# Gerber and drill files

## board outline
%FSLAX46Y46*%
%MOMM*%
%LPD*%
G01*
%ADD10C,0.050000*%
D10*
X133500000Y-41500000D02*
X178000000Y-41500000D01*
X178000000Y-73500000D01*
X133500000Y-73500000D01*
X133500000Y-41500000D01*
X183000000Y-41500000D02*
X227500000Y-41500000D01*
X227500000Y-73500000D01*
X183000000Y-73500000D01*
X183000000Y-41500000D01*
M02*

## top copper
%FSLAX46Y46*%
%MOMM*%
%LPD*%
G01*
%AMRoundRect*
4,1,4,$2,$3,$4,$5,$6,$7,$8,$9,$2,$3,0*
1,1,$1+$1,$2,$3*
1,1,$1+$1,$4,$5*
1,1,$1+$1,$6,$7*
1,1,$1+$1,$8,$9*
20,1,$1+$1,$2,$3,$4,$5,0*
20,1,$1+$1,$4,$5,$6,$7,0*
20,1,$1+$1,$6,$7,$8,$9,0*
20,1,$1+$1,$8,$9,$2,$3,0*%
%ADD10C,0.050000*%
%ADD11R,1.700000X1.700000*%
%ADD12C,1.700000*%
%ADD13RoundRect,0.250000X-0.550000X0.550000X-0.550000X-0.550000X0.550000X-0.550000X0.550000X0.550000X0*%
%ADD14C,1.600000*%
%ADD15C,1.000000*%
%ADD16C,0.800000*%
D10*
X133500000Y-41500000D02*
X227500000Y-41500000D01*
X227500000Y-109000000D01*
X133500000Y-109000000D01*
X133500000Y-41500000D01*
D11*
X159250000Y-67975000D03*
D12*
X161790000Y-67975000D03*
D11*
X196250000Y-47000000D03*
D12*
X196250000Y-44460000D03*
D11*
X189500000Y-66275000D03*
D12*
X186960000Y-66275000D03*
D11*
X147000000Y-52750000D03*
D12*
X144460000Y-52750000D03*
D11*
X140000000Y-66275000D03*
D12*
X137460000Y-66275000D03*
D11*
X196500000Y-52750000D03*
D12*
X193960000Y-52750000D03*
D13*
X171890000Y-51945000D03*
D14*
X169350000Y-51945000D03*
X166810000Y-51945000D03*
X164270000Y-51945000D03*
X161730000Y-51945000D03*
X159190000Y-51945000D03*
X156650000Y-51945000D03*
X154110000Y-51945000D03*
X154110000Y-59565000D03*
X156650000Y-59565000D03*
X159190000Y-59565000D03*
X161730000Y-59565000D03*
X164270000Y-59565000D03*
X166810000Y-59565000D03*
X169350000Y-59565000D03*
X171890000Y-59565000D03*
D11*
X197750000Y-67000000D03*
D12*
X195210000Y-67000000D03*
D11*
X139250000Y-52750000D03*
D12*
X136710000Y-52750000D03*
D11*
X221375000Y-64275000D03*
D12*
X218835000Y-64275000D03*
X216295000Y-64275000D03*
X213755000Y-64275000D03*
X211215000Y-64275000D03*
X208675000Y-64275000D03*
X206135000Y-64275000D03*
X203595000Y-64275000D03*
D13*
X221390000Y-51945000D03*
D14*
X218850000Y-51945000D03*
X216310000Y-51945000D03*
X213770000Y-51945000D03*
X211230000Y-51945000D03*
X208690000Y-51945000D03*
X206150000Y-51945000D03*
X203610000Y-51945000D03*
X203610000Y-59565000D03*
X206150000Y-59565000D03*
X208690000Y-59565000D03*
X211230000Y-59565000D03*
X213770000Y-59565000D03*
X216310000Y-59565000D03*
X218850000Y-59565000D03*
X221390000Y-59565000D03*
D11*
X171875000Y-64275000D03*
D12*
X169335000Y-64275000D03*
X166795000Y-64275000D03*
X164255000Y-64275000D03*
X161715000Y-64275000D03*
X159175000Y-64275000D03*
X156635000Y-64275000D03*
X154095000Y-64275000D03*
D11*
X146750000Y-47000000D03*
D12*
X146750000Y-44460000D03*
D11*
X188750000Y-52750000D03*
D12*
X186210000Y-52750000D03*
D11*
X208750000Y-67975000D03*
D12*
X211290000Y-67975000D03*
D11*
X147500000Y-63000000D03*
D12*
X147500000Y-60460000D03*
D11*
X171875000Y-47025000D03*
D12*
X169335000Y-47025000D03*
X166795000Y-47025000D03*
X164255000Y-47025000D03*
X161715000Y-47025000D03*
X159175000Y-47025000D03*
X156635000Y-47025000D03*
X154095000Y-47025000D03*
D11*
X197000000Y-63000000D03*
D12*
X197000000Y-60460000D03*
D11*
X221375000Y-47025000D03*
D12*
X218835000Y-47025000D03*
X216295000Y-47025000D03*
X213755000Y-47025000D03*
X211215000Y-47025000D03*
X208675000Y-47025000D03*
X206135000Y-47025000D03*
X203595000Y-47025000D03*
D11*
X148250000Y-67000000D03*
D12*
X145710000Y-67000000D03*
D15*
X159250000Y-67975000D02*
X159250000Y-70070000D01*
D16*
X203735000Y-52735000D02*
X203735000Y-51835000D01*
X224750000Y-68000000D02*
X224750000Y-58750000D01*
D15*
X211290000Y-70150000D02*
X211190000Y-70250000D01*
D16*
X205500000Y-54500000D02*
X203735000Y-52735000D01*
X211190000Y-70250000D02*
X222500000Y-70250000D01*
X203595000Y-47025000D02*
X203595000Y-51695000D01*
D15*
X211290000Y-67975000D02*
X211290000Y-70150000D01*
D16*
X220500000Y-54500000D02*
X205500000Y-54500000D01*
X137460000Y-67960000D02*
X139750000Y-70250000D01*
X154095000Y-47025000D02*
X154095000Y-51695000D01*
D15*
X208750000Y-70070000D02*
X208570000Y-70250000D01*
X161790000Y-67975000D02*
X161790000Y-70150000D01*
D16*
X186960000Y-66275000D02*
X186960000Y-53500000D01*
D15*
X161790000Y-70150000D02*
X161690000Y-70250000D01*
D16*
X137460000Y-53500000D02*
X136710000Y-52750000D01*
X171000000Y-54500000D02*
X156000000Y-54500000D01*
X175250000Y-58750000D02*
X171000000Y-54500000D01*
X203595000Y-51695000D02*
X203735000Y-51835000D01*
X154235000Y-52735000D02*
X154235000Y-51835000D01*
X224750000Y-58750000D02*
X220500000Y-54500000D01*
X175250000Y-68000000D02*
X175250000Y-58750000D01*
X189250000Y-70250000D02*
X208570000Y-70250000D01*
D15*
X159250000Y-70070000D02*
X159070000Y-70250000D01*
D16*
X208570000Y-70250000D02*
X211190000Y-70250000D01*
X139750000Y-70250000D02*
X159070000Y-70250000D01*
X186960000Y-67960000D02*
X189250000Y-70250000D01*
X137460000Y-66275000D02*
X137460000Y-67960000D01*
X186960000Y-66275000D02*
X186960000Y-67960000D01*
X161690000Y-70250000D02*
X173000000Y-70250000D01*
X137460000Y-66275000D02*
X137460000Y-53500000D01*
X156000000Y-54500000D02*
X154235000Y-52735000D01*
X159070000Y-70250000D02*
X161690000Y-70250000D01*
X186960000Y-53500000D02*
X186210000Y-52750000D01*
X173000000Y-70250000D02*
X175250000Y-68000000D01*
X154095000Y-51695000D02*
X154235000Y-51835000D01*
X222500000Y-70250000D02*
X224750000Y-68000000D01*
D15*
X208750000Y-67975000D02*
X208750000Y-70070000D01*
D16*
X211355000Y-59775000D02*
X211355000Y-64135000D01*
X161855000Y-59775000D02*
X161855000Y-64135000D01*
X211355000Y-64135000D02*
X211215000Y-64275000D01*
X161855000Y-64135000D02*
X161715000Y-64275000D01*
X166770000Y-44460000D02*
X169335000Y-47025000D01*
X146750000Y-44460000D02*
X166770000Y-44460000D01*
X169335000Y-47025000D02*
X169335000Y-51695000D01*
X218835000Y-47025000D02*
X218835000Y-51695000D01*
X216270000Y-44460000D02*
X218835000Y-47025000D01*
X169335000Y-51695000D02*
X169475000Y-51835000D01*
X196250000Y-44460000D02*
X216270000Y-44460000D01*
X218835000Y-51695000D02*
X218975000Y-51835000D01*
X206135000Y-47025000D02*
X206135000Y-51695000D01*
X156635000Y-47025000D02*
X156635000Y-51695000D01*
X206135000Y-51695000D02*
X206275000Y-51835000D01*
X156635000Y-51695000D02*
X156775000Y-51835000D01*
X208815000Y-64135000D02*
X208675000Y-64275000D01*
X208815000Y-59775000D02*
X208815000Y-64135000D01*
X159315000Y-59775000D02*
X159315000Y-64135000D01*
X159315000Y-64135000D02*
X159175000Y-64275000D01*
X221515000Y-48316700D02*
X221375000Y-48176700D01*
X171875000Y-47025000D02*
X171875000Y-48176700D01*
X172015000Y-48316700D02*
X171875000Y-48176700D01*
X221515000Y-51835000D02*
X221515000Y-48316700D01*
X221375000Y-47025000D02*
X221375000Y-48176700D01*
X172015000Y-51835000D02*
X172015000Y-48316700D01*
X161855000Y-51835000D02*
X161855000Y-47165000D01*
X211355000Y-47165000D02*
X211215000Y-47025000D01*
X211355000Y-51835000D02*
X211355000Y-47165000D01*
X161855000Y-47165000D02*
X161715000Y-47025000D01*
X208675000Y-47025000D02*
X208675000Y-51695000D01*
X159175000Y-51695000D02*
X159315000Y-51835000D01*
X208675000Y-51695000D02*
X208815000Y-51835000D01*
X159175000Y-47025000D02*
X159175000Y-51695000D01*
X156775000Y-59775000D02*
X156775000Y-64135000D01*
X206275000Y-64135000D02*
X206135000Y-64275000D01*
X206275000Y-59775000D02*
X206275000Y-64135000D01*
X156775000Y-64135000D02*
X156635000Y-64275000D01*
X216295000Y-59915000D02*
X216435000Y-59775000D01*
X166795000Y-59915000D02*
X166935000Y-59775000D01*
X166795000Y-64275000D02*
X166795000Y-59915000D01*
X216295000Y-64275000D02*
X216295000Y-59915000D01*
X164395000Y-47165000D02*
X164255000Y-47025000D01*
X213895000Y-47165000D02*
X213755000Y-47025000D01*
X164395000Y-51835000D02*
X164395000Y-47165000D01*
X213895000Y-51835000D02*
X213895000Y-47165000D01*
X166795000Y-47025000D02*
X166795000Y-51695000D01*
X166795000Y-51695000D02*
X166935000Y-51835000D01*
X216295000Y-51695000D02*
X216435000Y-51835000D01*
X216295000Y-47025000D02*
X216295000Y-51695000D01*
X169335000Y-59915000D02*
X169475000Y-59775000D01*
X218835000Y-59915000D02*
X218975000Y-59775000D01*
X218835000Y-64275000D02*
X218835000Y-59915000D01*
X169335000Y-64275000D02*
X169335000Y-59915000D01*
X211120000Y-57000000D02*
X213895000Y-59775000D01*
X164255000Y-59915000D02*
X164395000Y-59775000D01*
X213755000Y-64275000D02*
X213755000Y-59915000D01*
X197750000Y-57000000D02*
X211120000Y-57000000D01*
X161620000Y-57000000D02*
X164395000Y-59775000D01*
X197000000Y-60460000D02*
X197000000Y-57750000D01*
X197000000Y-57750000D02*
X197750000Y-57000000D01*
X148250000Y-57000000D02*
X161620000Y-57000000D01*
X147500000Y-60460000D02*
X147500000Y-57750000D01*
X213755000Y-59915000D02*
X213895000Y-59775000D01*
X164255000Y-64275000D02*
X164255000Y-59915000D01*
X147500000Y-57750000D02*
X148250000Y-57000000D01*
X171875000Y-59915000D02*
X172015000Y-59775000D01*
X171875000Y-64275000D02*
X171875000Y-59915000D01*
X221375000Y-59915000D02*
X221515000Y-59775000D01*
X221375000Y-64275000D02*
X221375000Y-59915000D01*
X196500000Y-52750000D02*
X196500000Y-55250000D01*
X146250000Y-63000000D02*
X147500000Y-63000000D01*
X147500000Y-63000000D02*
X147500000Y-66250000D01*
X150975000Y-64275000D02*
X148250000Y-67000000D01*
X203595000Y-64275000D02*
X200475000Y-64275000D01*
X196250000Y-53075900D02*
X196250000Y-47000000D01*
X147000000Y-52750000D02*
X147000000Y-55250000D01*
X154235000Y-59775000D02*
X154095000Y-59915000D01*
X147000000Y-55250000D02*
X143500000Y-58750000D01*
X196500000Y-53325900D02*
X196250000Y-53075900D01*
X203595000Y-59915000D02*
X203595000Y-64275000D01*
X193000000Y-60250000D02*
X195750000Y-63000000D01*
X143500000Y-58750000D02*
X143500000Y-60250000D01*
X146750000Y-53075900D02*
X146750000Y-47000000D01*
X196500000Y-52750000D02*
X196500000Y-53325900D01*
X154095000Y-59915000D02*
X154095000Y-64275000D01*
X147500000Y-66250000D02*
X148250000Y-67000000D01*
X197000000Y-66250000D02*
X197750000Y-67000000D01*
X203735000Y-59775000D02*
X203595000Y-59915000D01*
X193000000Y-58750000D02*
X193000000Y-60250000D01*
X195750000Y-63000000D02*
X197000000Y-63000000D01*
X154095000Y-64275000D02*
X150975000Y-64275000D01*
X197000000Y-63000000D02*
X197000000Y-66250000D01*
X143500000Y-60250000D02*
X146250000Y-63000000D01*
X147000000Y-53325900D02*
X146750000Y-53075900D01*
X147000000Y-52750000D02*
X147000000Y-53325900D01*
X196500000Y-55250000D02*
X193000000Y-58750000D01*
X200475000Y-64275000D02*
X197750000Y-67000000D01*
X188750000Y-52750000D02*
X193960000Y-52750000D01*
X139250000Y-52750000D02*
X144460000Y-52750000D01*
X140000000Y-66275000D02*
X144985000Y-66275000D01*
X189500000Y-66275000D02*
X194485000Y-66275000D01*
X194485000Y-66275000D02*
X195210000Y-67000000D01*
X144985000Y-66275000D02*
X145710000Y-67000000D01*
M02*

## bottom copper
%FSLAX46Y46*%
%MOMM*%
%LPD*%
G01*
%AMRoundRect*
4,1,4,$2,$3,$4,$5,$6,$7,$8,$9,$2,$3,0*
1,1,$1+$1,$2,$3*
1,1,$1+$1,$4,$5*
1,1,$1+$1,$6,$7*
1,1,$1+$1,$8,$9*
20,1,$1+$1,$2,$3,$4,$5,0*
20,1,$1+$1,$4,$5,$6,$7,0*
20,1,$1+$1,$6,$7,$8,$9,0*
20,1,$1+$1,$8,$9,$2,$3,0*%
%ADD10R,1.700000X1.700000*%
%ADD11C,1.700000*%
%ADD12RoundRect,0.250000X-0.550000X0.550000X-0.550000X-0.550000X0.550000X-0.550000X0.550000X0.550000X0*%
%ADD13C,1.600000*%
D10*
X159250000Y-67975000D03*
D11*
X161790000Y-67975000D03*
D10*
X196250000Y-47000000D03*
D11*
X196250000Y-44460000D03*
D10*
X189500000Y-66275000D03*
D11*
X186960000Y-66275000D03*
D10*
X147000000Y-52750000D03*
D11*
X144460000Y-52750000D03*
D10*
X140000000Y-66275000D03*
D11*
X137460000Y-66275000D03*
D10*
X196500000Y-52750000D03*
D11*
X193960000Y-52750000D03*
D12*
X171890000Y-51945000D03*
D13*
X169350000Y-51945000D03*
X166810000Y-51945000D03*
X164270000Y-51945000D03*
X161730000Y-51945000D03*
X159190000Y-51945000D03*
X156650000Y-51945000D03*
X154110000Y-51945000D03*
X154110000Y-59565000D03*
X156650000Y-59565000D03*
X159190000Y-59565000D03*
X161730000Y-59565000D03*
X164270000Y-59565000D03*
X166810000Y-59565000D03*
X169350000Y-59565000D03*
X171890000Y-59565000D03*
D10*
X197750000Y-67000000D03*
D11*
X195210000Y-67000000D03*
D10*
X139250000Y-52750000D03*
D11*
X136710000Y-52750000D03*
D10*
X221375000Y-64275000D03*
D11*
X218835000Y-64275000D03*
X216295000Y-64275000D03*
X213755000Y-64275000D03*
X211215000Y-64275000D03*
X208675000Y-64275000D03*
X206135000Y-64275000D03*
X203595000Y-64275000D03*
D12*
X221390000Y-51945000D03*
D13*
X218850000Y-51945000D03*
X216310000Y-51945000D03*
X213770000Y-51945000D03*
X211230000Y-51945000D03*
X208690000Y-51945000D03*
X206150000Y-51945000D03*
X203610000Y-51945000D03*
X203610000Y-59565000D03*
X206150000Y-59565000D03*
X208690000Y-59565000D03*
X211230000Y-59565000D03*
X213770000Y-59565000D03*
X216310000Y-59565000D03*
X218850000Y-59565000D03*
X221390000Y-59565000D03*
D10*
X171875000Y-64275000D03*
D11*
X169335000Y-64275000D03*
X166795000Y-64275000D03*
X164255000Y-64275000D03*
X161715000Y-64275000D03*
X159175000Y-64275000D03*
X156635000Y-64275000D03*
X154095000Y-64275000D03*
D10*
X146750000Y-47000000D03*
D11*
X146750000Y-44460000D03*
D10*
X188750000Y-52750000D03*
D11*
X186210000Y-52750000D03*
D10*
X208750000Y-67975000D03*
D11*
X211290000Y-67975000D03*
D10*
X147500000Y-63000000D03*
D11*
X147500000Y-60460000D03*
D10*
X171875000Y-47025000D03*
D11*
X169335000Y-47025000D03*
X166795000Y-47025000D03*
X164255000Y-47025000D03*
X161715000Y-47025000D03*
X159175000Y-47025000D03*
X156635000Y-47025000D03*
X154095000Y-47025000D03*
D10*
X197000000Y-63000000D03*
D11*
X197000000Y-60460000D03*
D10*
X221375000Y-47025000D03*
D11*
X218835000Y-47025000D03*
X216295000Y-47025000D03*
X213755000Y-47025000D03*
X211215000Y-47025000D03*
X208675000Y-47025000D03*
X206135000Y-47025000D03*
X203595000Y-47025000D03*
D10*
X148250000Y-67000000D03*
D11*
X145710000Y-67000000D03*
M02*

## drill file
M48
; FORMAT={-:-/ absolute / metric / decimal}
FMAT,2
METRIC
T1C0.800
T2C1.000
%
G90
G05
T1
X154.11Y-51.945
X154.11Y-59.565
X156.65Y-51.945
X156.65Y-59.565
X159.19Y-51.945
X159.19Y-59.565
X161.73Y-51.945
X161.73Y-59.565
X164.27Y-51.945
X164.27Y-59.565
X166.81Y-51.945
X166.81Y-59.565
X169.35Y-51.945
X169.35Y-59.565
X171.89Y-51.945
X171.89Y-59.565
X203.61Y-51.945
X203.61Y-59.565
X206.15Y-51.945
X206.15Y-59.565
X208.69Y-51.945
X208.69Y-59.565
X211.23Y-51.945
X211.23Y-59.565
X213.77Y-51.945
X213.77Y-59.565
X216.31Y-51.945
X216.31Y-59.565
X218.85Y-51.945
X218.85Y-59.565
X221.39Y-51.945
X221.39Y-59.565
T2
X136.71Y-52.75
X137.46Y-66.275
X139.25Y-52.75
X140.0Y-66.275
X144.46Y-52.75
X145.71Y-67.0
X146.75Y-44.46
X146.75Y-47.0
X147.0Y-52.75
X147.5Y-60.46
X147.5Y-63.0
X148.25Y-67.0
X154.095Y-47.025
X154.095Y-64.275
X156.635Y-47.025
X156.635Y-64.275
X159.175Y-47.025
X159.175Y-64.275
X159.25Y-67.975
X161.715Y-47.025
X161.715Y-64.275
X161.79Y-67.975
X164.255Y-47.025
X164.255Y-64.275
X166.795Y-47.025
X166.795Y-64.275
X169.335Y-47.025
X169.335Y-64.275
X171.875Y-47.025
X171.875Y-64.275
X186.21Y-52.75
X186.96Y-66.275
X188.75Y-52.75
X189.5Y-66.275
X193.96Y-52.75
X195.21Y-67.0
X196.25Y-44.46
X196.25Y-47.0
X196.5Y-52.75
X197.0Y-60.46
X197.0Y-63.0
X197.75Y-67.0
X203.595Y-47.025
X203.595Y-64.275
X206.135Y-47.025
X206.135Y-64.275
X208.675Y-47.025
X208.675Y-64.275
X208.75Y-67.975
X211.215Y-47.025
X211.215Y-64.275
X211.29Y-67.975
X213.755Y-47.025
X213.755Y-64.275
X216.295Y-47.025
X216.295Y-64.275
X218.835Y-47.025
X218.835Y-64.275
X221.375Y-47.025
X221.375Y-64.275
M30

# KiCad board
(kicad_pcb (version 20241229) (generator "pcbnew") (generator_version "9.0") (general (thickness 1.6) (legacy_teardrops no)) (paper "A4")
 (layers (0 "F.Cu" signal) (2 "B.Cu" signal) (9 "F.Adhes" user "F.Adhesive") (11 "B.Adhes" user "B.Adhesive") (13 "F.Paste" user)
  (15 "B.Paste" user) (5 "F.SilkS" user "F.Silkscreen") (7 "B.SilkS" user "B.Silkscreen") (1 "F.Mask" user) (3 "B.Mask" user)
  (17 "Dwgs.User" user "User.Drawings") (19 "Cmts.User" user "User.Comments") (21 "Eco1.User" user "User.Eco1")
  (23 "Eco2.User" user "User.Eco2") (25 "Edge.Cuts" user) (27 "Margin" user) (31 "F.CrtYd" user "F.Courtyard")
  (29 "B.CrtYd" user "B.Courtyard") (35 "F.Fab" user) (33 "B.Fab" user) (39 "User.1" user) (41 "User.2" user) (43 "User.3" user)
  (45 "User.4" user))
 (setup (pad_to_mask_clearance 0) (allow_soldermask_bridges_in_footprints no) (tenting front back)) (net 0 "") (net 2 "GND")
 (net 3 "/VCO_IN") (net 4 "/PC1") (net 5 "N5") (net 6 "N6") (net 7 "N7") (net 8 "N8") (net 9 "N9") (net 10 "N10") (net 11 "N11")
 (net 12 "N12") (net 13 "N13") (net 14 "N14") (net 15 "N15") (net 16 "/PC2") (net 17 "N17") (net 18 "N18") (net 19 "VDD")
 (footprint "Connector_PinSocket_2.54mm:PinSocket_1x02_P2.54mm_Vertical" (layer "F.Cu") (at 159.25 67.975 90)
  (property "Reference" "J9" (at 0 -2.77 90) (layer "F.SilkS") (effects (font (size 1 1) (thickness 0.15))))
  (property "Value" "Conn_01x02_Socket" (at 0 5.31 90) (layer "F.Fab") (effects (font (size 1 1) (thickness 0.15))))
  (pad "1" thru_hole rect (at 0 0 90) (size 1.7 1.7) (drill 1) (layers "*.Cu" "*.Mask") (remove_unused_layers no) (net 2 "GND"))
  (pad "2" thru_hole circle (at 0 2.54 90) (size 1.7 1.7) (drill 1) (layers "*.Cu" "*.Mask") (remove_unused_layers no) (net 2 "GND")))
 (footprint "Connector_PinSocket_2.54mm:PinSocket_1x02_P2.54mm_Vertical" (layer "F.Cu") (at 196.25 47 180)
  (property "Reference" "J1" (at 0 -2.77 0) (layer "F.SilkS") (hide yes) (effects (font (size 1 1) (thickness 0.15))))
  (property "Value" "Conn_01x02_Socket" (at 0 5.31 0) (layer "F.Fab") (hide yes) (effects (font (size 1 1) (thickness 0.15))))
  (pad "1" thru_hole rect (at 0 0 180) (size 1.7 1.7) (drill 1) (layers "*.Cu" "*.Mask") (remove_unused_layers no) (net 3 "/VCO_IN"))
  (pad "2" thru_hole circle (at 0 2.54 180) (size 1.7 1.7) (drill 1) (layers "*.Cu" "*.Mask") (remove_unused_layers no) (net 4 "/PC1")))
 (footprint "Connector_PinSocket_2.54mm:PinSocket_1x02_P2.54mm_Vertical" (layer "F.Cu") (at 189.5 66.275 -90)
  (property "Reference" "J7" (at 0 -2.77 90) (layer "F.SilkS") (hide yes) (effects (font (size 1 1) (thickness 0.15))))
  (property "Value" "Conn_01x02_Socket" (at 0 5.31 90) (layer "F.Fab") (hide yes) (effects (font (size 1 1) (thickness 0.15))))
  (pad "1" thru_hole rect (at 0 0 270) (size 1.7 1.7) (drill 1) (layers "*.Cu" "*.Mask") (remove_unused_layers no) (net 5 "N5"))
  (pad "2" thru_hole circle (at 0 2.54 270) (size 1.7 1.7) (drill 1) (layers "*.Cu" "*.Mask") (remove_unused_layers no) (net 2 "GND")))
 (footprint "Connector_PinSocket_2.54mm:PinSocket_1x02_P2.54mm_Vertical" (layer "F.Cu") (at 147 52.75 -90)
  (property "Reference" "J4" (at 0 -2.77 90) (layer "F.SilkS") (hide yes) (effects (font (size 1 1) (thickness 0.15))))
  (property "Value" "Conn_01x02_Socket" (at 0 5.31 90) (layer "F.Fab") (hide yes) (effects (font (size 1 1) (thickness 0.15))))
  (pad "1" thru_hole rect (at 0 0 270) (size 1.7 1.7) (drill 1) (layers "*.Cu" "*.Mask") (remove_unused_layers no) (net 3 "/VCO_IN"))
  (pad "2" thru_hole circle (at 0 2.54 270) (size 1.7 1.7) (drill 1) (layers "*.Cu" "*.Mask") (remove_unused_layers no) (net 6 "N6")))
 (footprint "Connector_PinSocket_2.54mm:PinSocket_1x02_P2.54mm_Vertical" (layer "F.Cu") (at 140 66.275 -90)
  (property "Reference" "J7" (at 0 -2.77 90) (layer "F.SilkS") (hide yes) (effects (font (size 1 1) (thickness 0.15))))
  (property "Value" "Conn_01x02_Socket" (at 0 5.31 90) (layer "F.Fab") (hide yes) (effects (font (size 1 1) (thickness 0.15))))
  (pad "1" thru_hole rect (at 0 0 270) (size 1.7 1.7) (drill 1) (layers "*.Cu" "*.Mask") (remove_unused_layers no) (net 5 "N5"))
  (pad "2" thru_hole circle (at 0 2.54 270) (size 1.7 1.7) (drill 1) (layers "*.Cu" "*.Mask") (remove_unused_layers no) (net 2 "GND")))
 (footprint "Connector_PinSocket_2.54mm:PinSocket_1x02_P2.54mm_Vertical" (layer "F.Cu") (at 196.5 52.75 -90)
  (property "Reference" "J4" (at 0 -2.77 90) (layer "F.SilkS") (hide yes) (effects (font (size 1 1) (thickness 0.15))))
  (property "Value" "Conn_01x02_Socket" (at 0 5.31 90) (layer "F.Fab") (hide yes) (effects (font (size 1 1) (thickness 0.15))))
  (pad "1" thru_hole rect (at 0 0 270) (size 1.7 1.7) (drill 1) (layers "*.Cu" "*.Mask") (remove_unused_layers no) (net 3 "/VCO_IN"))
  (pad "2" thru_hole circle (at 0 2.54 270) (size 1.7 1.7) (drill 1) (layers "*.Cu" "*.Mask") (remove_unused_layers no) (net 6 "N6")))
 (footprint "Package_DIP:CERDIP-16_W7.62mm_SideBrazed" (layer "F.Cu") (at 171.89 51.945 -90)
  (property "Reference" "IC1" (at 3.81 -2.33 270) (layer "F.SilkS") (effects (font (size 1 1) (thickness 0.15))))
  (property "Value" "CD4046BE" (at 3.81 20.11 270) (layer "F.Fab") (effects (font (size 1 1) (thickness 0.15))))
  (pad "1" thru_hole roundrect (at 0 0 270) (size 1.6 1.6) (drill 0.8) (layers "*.Cu" "*.Mask") (remove_unused_layers no)
   (roundrect_rratio 0.15625) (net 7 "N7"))
  (pad "2" thru_hole circle (at 0 2.54 270) (size 1.6 1.6) (drill 0.8) (layers "*.Cu" "*.Mask") (remove_unused_layers no) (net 4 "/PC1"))
  (pad "3" thru_hole circle (at 0 5.08 270) (size 1.6 1.6) (drill 0.8) (layers "*.Cu" "*.Mask") (remove_unused_layers no) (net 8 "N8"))
  (pad "4" thru_hole circle (at 0 7.62 270) (size 1.6 1.6) (drill 0.8) (layers "*.Cu" "*.Mask") (remove_unused_layers no) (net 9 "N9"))
  (pad "5" thru_hole circle (at 0 10.16 270) (size 1.6 1.6) (drill 0.8) (layers "*.Cu" "*.Mask") (remove_unused_layers no) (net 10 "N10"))
  (pad "6" thru_hole circle (at 0 12.7 270) (size 1.6 1.6) (drill 0.8) (layers "*.Cu" "*.Mask") (remove_unused_layers no) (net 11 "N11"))
  (pad "7" thru_hole circle (at 0 15.24 270) (size 1.6 1.6) (drill 0.8) (layers "*.Cu" "*.Mask") (remove_unused_layers no) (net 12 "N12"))
  (pad "8" thru_hole circle (at 0 17.78 270) (size 1.6 1.6) (drill 0.8) (layers "*.Cu" "*.Mask") (remove_unused_layers no) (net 2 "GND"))
  (pad "9" thru_hole circle (at 7.62 17.78 270) (size 1.6 1.6) (drill 0.8) (layers "*.Cu" "*.Mask") (remove_unused_layers no)
   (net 3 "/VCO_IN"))
  (pad "10" thru_hole circle (at 7.62 15.24 270) (size 1.6 1.6) (drill 0.8) (layers "*.Cu" "*.Mask") (remove_unused_layers no)
   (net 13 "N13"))
  (pad "11" thru_hole circle (at 7.62 12.7 270) (size 1.6 1.6) (drill 0.8) (layers "*.Cu" "*.Mask") (remove_unused_layers no) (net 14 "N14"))
  (pad "12" thru_hole circle (at 7.62 10.16 270) (size 1.6 1.6) (drill 0.8) (layers "*.Cu" "*.Mask") (remove_unused_layers no)
   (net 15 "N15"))
  (pad "13" thru_hole circle (at 7.62 7.62 270) (size 1.6 1.6) (drill 0.8) (layers "*.Cu" "*.Mask") (remove_unused_layers no)
   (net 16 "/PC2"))
  (pad "14" thru_hole circle (at 7.62 5.08 270) (size 1.6 1.6) (drill 0.8) (layers "*.Cu" "*.Mask") (remove_unused_layers no) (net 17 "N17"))
  (pad "15" thru_hole circle (at 7.62 2.54 270) (size 1.6 1.6) (drill 0.8) (layers "*.Cu" "*.Mask") (remove_unused_layers no) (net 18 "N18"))
  (pad "16" thru_hole circle (at 7.62 0 270) (size 1.6 1.6) (drill 0.8) (layers "*.Cu" "*.Mask") (remove_unused_layers no) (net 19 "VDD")))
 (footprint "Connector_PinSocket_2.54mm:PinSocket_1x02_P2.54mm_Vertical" (layer "F.Cu") (at 197.75 67 -90)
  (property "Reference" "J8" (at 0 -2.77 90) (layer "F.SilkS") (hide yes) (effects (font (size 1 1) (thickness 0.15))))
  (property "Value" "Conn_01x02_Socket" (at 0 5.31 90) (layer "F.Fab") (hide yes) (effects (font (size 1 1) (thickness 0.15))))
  (pad "1" thru_hole rect (at 0 0 270) (size 1.7 1.7) (drill 1) (layers "*.Cu" "*.Mask") (remove_unused_layers no) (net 3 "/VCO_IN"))
  (pad "2" thru_hole circle (at 0 2.54 270) (size 1.7 1.7) (drill 1) (layers "*.Cu" "*.Mask") (remove_unused_layers no) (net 5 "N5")))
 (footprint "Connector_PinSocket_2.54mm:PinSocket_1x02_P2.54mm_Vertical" (layer "F.Cu") (at 139.25 52.75 -90)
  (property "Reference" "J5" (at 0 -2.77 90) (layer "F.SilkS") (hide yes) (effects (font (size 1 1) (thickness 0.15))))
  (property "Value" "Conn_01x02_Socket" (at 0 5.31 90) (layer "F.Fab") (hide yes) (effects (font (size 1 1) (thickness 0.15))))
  (pad "1" thru_hole rect (at 0 0 270) (size 1.7 1.7) (drill 1) (layers "*.Cu" "*.Mask") (remove_unused_layers no) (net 6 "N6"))
  (pad "2" thru_hole circle (at 0 2.54 270) (size 1.7 1.7) (drill 1) (layers "*.Cu" "*.Mask") (remove_unused_layers no) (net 2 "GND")))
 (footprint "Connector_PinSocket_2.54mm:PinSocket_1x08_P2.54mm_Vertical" (layer "F.Cu") (at 221.375 64.275 -90)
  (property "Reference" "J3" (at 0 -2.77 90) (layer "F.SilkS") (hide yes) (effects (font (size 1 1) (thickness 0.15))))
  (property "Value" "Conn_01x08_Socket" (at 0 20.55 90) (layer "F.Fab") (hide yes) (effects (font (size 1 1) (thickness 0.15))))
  (pad "1" thru_hole rect (at 0 0 270) (size 1.7 1.7) (drill 1) (layers "*.Cu" "*.Mask") (remove_unused_layers no) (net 19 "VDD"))
  (pad "2" thru_hole circle (at 0 2.54 270) (size 1.7 1.7) (drill 1) (layers "*.Cu" "*.Mask") (remove_unused_layers no) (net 18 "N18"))
  (pad "3" thru_hole circle (at 0 5.08 270) (size 1.7 1.7) (drill 1) (layers "*.Cu" "*.Mask") (remove_unused_layers no) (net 17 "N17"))
  (pad "4" thru_hole circle (at 0 7.62 270) (size 1.7 1.7) (drill 1) (layers "*.Cu" "*.Mask") (remove_unused_layers no) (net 16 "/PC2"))
  (pad "5" thru_hole circle (at 0 10.16 270) (size 1.7 1.7) (drill 1) (layers "*.Cu" "*.Mask") (remove_unused_layers no) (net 15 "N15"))
  (pad "6" thru_hole circle (at 0 12.7 270) (size 1.7 1.7) (drill 1) (layers "*.Cu" "*.Mask") (remove_unused_layers no) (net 14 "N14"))
  (pad "7" thru_hole circle (at 0 15.24 270) (size 1.7 1.7) (drill 1) (layers "*.Cu" "*.Mask") (remove_unused_layers no) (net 13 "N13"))
  (pad "8" thru_hole circle (at 0 17.78 270) (size 1.7 1.7) (drill 1) (layers "*.Cu" "*.Mask") (remove_unused_layers no) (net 3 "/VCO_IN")))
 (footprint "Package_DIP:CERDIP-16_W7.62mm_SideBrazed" (layer "F.Cu") (at 221.39 51.945 -90)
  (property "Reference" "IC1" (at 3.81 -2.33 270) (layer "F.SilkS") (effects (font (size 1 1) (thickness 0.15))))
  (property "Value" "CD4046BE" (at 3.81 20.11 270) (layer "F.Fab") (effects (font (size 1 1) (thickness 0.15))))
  (pad "1" thru_hole roundrect (at 0 0 270) (size 1.6 1.6) (drill 0.8) (layers "*.Cu" "*.Mask") (remove_unused_layers no)
   (roundrect_rratio 0.15625) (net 7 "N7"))
  (pad "2" thru_hole circle (at 0 2.54 270) (size 1.6 1.6) (drill 0.8) (layers "*.Cu" "*.Mask") (remove_unused_layers no) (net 4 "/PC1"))
  (pad "3" thru_hole circle (at 0 5.08 270) (size 1.6 1.6) (drill 0.8) (layers "*.Cu" "*.Mask") (remove_unused_layers no) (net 8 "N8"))
  (pad "4" thru_hole circle (at 0 7.62 270) (size 1.6 1.6) (drill 0.8) (layers "*.Cu" "*.Mask") (remove_unused_layers no) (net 9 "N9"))
  (pad "5" thru_hole circle (at 0 10.16 270) (size 1.6 1.6) (drill 0.8) (layers "*.Cu" "*.Mask") (remove_unused_layers no) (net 10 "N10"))
  (pad "6" thru_hole circle (at 0 12.7 270) (size 1.6 1.6) (drill 0.8) (layers "*.Cu" "*.Mask") (remove_unused_layers no) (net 11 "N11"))
  (pad "7" thru_hole circle (at 0 15.24 270) (size 1.6 1.6) (drill 0.8) (layers "*.Cu" "*.Mask") (remove_unused_layers no) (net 12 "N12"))
  (pad "8" thru_hole circle (at 0 17.78 270) (size 1.6 1.6) (drill 0.8) (layers "*.Cu" "*.Mask") (remove_unused_layers no) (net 2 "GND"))
  (pad "9" thru_hole circle (at 7.62 17.78 270) (size 1.6 1.6) (drill 0.8) (layers "*.Cu" "*.Mask") (remove_unused_layers no)
   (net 3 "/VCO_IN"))
  (pad "10" thru_hole circle (at 7.62 15.24 270) (size 1.6 1.6) (drill 0.8) (layers "*.Cu" "*.Mask") (remove_unused_layers no)
   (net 13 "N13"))
  (pad "11" thru_hole circle (at 7.62 12.7 270) (size 1.6 1.6) (drill 0.8) (layers "*.Cu" "*.Mask") (remove_unused_layers no) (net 14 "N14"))
  (pad "12" thru_hole circle (at 7.62 10.16 270) (size 1.6 1.6) (drill 0.8) (layers "*.Cu" "*.Mask") (remove_unused_layers no)
   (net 15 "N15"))
  (pad "13" thru_hole circle (at 7.62 7.62 270) (size 1.6 1.6) (drill 0.8) (layers "*.Cu" "*.Mask") (remove_unused_layers no)
   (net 16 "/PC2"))
  (pad "14" thru_hole circle (at 7.62 5.08 270) (size 1.6 1.6) (drill 0.8) (layers "*.Cu" "*.Mask") (remove_unused_layers no) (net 17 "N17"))
  (pad "15" thru_hole circle (at 7.62 2.54 270) (size 1.6 1.6) (drill 0.8) (layers "*.Cu" "*.Mask") (remove_unused_layers no) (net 18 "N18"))
  (pad "16" thru_hole circle (at 7.62 0 270) (size 1.6 1.6) (drill 0.8) (layers "*.Cu" "*.Mask") (remove_unused_layers no) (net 19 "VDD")))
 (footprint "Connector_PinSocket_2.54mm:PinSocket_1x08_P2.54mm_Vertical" (layer "F.Cu") (at 171.875 64.275 -90)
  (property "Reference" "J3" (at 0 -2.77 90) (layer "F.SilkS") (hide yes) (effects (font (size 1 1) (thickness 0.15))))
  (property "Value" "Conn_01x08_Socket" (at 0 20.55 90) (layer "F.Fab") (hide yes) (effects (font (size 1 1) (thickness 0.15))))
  (pad "1" thru_hole rect (at 0 0 270) (size 1.7 1.7) (drill 1) (layers "*.Cu" "*.Mask") (remove_unused_layers no) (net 19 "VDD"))
  (pad "2" thru_hole circle (at 0 2.54 270) (size 1.7 1.7) (drill 1) (layers "*.Cu" "*.Mask") (remove_unused_layers no) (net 18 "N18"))
  (pad "3" thru_hole circle (at 0 5.08 270) (size 1.7 1.7) (drill 1) (layers "*.Cu" "*.Mask") (remove_unused_layers no) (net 17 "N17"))
  (pad "4" thru_hole circle (at 0 7.62 270) (size 1.7 1.7) (drill 1) (layers "*.Cu" "*.Mask") (remove_unused_layers no) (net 16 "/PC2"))
  (pad "5" thru_hole circle (at 0 10.16 270) (size 1.7 1.7) (drill 1) (layers "*.Cu" "*.Mask") (remove_unused_layers no) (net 15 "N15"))
  (pad "6" thru_hole circle (at 0 12.7 270) (size 1.7 1.7) (drill 1) (layers "*.Cu" "*.Mask") (remove_unused_layers no) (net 14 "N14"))
  (pad "7" thru_hole circle (at 0 15.24 270) (size 1.7 1.7) (drill 1) (layers "*.Cu" "*.Mask") (remove_unused_layers no) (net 13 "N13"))
  (pad "8" thru_hole circle (at 0 17.78 270) (size 1.7 1.7) (drill 1) (layers "*.Cu" "*.Mask") (remove_unused_layers no) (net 3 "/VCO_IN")))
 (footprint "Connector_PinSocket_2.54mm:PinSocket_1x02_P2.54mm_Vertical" (layer "F.Cu") (at 146.75 47 180)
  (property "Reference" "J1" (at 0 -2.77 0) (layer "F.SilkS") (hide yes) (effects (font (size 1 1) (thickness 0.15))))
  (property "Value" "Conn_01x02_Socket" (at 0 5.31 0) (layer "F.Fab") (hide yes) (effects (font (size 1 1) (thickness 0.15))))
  (pad "1" thru_hole rect (at 0 0 180) (size 1.7 1.7) (drill 1) (layers "*.Cu" "*.Mask") (remove_unused_layers no) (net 3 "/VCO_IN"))
  (pad "2" thru_hole circle (at 0 2.54 180) (size 1.7 1.7) (drill 1) (layers "*.Cu" "*.Mask") (remove_unused_layers no) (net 4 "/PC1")))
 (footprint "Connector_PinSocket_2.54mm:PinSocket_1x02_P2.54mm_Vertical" (layer "F.Cu") (at 188.75 52.75 -90)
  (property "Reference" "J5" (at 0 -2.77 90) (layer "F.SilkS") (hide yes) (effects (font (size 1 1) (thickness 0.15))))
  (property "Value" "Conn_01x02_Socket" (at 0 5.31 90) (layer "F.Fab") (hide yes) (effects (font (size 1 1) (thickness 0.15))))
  (pad "1" thru_hole rect (at 0 0 270) (size 1.7 1.7) (drill 1) (layers "*.Cu" "*.Mask") (remove_unused_layers no) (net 6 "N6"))
  (pad "2" thru_hole circle (at 0 2.54 270) (size 1.7 1.7) (drill 1) (layers "*.Cu" "*.Mask") (remove_unused_layers no) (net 2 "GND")))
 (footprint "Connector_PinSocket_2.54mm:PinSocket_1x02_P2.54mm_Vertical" (layer "F.Cu") (at 208.75 67.975 90)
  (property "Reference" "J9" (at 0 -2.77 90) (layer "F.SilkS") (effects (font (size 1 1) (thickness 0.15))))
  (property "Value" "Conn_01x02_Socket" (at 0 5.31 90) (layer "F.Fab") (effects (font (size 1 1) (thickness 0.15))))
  (pad "1" thru_hole rect (at 0 0 90) (size 1.7 1.7) (drill 1) (layers "*.Cu" "*.Mask") (remove_unused_layers no) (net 2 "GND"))
  (pad "2" thru_hole circle (at 0 2.54 90) (size 1.7 1.7) (drill 1) (layers "*.Cu" "*.Mask") (remove_unused_layers no) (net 2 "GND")))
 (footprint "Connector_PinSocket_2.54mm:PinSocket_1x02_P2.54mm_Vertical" (layer "F.Cu") (at 147.5 63 180)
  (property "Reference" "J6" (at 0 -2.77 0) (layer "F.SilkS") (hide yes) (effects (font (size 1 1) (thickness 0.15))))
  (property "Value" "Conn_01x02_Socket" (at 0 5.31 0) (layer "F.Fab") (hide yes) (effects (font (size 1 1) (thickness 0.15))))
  (pad "1" thru_hole rect (at 0 0 180) (size 1.7 1.7) (drill 1) (layers "*.Cu" "*.Mask") (remove_unused_layers no) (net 3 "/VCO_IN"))
  (pad "2" thru_hole circle (at 0 2.54 180) (size 1.7 1.7) (drill 1) (layers "*.Cu" "*.Mask") (remove_unused_layers no) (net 16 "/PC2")))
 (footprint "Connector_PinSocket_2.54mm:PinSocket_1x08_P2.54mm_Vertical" (layer "F.Cu") (at 171.875 47.025 -90)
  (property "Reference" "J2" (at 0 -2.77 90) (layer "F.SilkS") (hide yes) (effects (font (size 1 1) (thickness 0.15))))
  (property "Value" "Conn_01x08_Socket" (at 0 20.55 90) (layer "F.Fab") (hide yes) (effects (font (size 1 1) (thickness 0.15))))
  (pad "1" thru_hole rect (at 0 0 270) (size 1.7 1.7) (drill 1) (layers "*.Cu" "*.Mask") (remove_unused_layers no) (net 7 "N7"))
  (pad "2" thru_hole circle (at 0 2.54 270) (size 1.7 1.7) (drill 1) (layers "*.Cu" "*.Mask") (remove_unused_layers no) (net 4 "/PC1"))
  (pad "3" thru_hole circle (at 0 5.08 270) (size 1.7 1.7) (drill 1) (layers "*.Cu" "*.Mask") (remove_unused_layers no) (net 8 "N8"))
  (pad "4" thru_hole circle (at 0 7.62 270) (size 1.7 1.7) (drill 1) (layers "*.Cu" "*.Mask") (remove_unused_layers no) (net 9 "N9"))
  (pad "5" thru_hole circle (at 0 10.16 270) (size 1.7 1.7) (drill 1) (layers "*.Cu" "*.Mask") (remove_unused_layers no) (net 10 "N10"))
  (pad "6" thru_hole circle (at 0 12.7 270) (size 1.7 1.7) (drill 1) (layers "*.Cu" "*.Mask") (remove_unused_layers no) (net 11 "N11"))
  (pad "7" thru_hole circle (at 0 15.24 270) (size 1.7 1.7) (drill 1) (layers "*.Cu" "*.Mask") (remove_unused_layers no) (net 12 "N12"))
  (pad "8" thru_hole circle (at 0 17.78 270) (size 1.7 1.7) (drill 1) (layers "*.Cu" "*.Mask") (remove_unused_layers no) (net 2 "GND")))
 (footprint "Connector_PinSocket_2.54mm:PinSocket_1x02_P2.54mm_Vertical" (layer "F.Cu") (at 197 63 180)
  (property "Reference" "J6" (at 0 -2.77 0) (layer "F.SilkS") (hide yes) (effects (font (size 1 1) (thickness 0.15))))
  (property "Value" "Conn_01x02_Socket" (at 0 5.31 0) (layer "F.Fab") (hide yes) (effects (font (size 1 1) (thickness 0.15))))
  (pad "1" thru_hole rect (at 0 0 180) (size 1.7 1.7) (drill 1) (layers "*.Cu" "*.Mask") (remove_unused_layers no) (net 3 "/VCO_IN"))
  (pad "2" thru_hole circle (at 0 2.54 180) (size 1.7 1.7) (drill 1) (layers "*.Cu" "*.Mask") (remove_unused_layers no) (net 16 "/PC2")))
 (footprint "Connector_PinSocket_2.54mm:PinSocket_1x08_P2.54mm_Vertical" (layer "F.Cu") (at 221.375 47.025 -90)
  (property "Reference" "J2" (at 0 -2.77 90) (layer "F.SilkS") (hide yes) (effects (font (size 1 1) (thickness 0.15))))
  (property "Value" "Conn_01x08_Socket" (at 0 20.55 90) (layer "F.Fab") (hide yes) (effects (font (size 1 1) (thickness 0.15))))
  (pad "1" thru_hole rect (at 0 0 270) (size 1.7 1.7) (drill 1) (layers "*.Cu" "*.Mask") (remove_unused_layers no) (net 7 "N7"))
  (pad "2" thru_hole circle (at 0 2.54 270) (size 1.7 1.7) (drill 1) (layers "*.Cu" "*.Mask") (remove_unused_layers no) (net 4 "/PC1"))
  (pad "3" thru_hole circle (at 0 5.08 270) (size 1.7 1.7) (drill 1) (layers "*.Cu" "*.Mask") (remove_unused_layers no) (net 8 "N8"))
  (pad "4" thru_hole circle (at 0 7.62 270) (size 1.7 1.7) (drill 1) (layers "*.Cu" "*.Mask") (remove_unused_layers no) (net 9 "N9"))
  (pad "5" thru_hole circle (at 0 10.16 270) (size 1.7 1.7) (drill 1) (layers "*.Cu" "*.Mask") (remove_unused_layers no) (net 10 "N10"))
  (pad "6" thru_hole circle (at 0 12.7 270) (size 1.7 1.7) (drill 1) (layers "*.Cu" "*.Mask") (remove_unused_layers no) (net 11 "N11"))
  (pad "7" thru_hole circle (at 0 15.24 270) (size 1.7 1.7) (drill 1) (layers "*.Cu" "*.Mask") (remove_unused_layers no) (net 12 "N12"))
  (pad "8" thru_hole circle (at 0 17.78 270) (size 1.7 1.7) (drill 1) (layers "*.Cu" "*.Mask") (remove_unused_layers no) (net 2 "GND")))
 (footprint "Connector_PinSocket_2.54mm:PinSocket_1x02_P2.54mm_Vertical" (layer "F.Cu") (at 148.25 67 -90)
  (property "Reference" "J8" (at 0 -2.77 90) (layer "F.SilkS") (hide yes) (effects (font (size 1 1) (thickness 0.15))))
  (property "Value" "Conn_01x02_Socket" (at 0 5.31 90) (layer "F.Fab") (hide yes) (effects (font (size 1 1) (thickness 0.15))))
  (pad "1" thru_hole rect (at 0 0 270) (size 1.7 1.7) (drill 1) (layers "*.Cu" "*.Mask") (remove_unused_layers no) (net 3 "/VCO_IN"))
  (pad "2" thru_hole circle (at 0 2.54 270) (size 1.7 1.7) (drill 1) (layers "*.Cu" "*.Mask") (remove_unused_layers no) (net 5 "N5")))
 (gr_rect (start 133.5 41.5) (end 227.5 109) (stroke (width 0.05) (type solid)) (fill no) (layer "F.Cu"))
 (gr_rect (start 133.5 41.5) (end 178 73.5) (stroke (width 0.05) (type default)) (fill no) (layer "Edge.Cuts"))
 (gr_rect (start 183 41.5) (end 227.5 73.5) (stroke (width 0.05) (type default)) (fill no) (layer "Edge.Cuts"))
 (segment (start 159.25 67.975) (end 159.25 70.07) (width 1) (layer "F.Cu") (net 2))
 (segment (start 203.735 52.735) (end 203.735 51.835) (width 0.8) (layer "F.Cu") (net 2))
 (segment (start 224.75 68) (end 224.75 58.75) (width 0.8) (layer "F.Cu") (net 2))
 (segment (start 211.29 70.15) (end 211.19 70.25) (width 1) (layer "F.Cu") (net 2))
 (segment (start 205.5 54.5) (end 203.735 52.735) (width 0.8) (layer "F.Cu") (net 2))
 (segment (start 211.19 70.25) (end 222.5 70.25) (width 0.8) (layer "F.Cu") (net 2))
 (segment (start 203.595 47.025) (end 203.595 51.695) (width 0.8) (layer "F.Cu") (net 2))
 (segment (start 211.29 67.975) (end 211.29 70.15) (width 1) (layer "F.Cu") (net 2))
 (segment (start 220.5 54.5) (end 205.5 54.5) (width 0.8) (layer "F.Cu") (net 2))
 (segment (start 137.46 67.96) (end 139.75 70.25) (width 0.8) (layer "F.Cu") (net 2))
 (segment (start 154.095 47.025) (end 154.095 51.695) (width 0.8) (layer "F.Cu") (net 2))
 (segment (start 208.75 70.07) (end 208.57 70.25) (width 1) (layer "F.Cu") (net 2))
 (segment (start 161.79 67.975) (end 161.79 70.15) (width 1) (layer "F.Cu") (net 2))
 (segment (start 186.96 66.275) (end 186.96 53.5) (width 0.8) (layer "F.Cu") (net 2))
 (segment (start 161.79 70.15) (end 161.69 70.25) (width 1) (layer "F.Cu") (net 2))
 (segment (start 137.46 53.5) (end 136.71 52.75) (width 0.8) (layer "F.Cu") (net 2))
 (segment (start 171 54.5) (end 156 54.5) (width 0.8) (layer "F.Cu") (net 2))
 (segment (start 175.25 58.75) (end 171 54.5) (width 0.8) (layer "F.Cu") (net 2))
 (segment (start 203.595 51.695) (end 203.735 51.835) (width 0.8) (layer "F.Cu") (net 2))
 (segment (start 154.235 52.735) (end 154.235 51.835) (width 0.8) (layer "F.Cu") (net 2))
 (segment (start 224.75 58.75) (end 220.5 54.5) (width 0.8) (layer "F.Cu") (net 2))
 (segment (start 175.25 68) (end 175.25 58.75) (width 0.8) (layer "F.Cu") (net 2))
 (segment (start 189.25 70.25) (end 208.57 70.25) (width 0.8) (layer "F.Cu") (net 2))
 (segment (start 159.25 70.07) (end 159.07 70.25) (width 1) (layer "F.Cu") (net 2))
 (segment (start 208.57 70.25) (end 211.19 70.25) (width 0.8) (layer "F.Cu") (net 2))
 (segment (start 139.75 70.25) (end 159.07 70.25) (width 0.8) (layer "F.Cu") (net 2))
 (segment (start 186.96 67.96) (end 189.25 70.25) (width 0.8) (layer "F.Cu") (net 2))
 (segment (start 137.46 66.275) (end 137.46 67.96) (width 0.8) (layer "F.Cu") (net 2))
 (segment (start 186.96 66.275) (end 186.96 67.96) (width 0.8) (layer "F.Cu") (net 2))
 (segment (start 161.69 70.25) (end 173 70.25) (width 0.8) (layer "F.Cu") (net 2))
 (segment (start 137.46 66.275) (end 137.46 53.5) (width 0.8) (layer "F.Cu") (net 2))
 (segment (start 156 54.5) (end 154.235 52.735) (width 0.8) (layer "F.Cu") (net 2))
 (segment (start 159.07 70.25) (end 161.69 70.25) (width 0.8) (layer "F.Cu") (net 2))
 (segment (start 186.96 53.5) (end 186.21 52.75) (width 0.8) (layer "F.Cu") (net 2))
 (segment (start 173 70.25) (end 175.25 68) (width 0.8) (layer "F.Cu") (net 2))
 (segment (start 154.095 51.695) (end 154.235 51.835) (width 0.8) (layer "F.Cu") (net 2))
 (segment (start 222.5 70.25) (end 224.75 68) (width 0.8) (layer "F.Cu") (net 2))
 (segment (start 208.75 67.975) (end 208.75 70.07) (width 1) (layer "F.Cu") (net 2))
 (segment (start 211.355 59.775) (end 211.355 64.135) (width 0.8) (layer "F.Cu") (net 15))
 (segment (start 161.855 59.775) (end 161.855 64.135) (width 0.8) (layer "F.Cu") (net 15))
 (segment (start 211.355 64.135) (end 211.215 64.275) (width 0.8) (layer "F.Cu") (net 15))
 (segment (start 161.855 64.135) (end 161.715 64.275) (width 0.8) (layer "F.Cu") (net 15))
 (segment (start 166.77 44.46) (end 169.335 47.025) (width 0.8) (layer "F.Cu") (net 4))
 (segment (start 146.75 44.46) (end 166.77 44.46) (width 0.8) (layer "F.Cu") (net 4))
 (segment (start 169.335 47.025) (end 169.335 51.695) (width 0.8) (layer "F.Cu") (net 4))
 (segment (start 218.835 47.025) (end 218.835 51.695) (width 0.8) (layer "F.Cu") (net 4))
 (segment (start 216.27 44.46) (end 218.835 47.025) (width 0.8) (layer "F.Cu") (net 4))
 (segment (start 169.335 51.695) (end 169.475 51.835) (width 0.8) (layer "F.Cu") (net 4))
 (segment (start 196.25 44.46) (end 216.27 44.46) (width 0.8) (layer "F.Cu") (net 4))
 (segment (start 218.835 51.695) (end 218.975 51.835) (width 0.8) (layer "F.Cu") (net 4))
 (segment (start 206.135 47.025) (end 206.135 51.695) (width 0.8) (layer "F.Cu") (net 12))
 (segment (start 156.635 47.025) (end 156.635 51.695) (width 0.8) (layer "F.Cu") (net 12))
 (segment (start 206.135 51.695) (end 206.275 51.835) (width 0.8) (layer "F.Cu") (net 12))
 (segment (start 156.635 51.695) (end 156.775 51.835) (width 0.8) (layer "F.Cu") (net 12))
 (segment (start 208.815 64.135) (end 208.675 64.275) (width 0.8) (layer "F.Cu") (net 14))
 (segment (start 208.815 59.775) (end 208.815 64.135) (width 0.8) (layer "F.Cu") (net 14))
 (segment (start 159.315 59.775) (end 159.315 64.135) (width 0.8) (layer "F.Cu") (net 14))
 (segment (start 159.315 64.135) (end 159.175 64.275) (width 0.8) (layer "F.Cu") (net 14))
 (segment (start 221.515 48.3167) (end 221.375 48.1767) (width 0.8) (layer "F.Cu") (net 7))
 (segment (start 171.875 47.025) (end 171.875 48.1767) (width 0.8) (layer "F.Cu") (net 7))
 (segment (start 172.015 48.3167) (end 171.875 48.1767) (width 0.8) (layer "F.Cu") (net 7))
 (segment (start 221.515 51.835) (end 221.515 48.3167) (width 0.8) (layer "F.Cu") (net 7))
 (segment (start 221.375 47.025) (end 221.375 48.1767) (width 0.8) (layer "F.Cu") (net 7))
 (segment (start 172.015 51.835) (end 172.015 48.3167) (width 0.8) (layer "F.Cu") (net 7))
 (segment (start 161.855 51.835) (end 161.855 47.165) (width 0.8) (layer "F.Cu") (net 10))
 (segment (start 211.355 47.165) (end 211.215 47.025) (width 0.8) (layer "F.Cu") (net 10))
 (segment (start 211.355 51.835) (end 211.355 47.165) (width 0.8) (layer "F.Cu") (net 10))
 (segment (start 161.855 47.165) (end 161.715 47.025) (width 0.8) (layer "F.Cu") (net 10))
 (segment (start 208.675 47.025) (end 208.675 51.695) (width 0.8) (layer "F.Cu") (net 11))
 (segment (start 159.175 51.695) (end 159.315 51.835) (width 0.8) (layer "F.Cu") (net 11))
 (segment (start 208.675 51.695) (end 208.815 51.835) (width 0.8) (layer "F.Cu") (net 11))
 (segment (start 159.175 47.025) (end 159.175 51.695) (width 0.8) (layer "F.Cu") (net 11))
 (segment (start 156.775 59.775) (end 156.775 64.135) (width 0.8) (layer "F.Cu") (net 13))
 (segment (start 206.275 64.135) (end 206.135 64.275) (width 0.8) (layer "F.Cu") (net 13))
 (segment (start 206.275 59.775) (end 206.275 64.135) (width 0.8) (layer "F.Cu") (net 13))
 (segment (start 156.775 64.135) (end 156.635 64.275) (width 0.8) (layer "F.Cu") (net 13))
 (segment (start 216.295 59.915) (end 216.435 59.775) (width 0.8) (layer "F.Cu") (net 17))
 (segment (start 166.795 59.915) (end 166.935 59.775) (width 0.8) (layer "F.Cu") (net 17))
 (segment (start 166.795 64.275) (end 166.795 59.915) (width 0.8) (layer "F.Cu") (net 17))
 (segment (start 216.295 64.275) (end 216.295 59.915) (width 0.8) (layer "F.Cu") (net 17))
 (segment (start 164.395 47.165) (end 164.255 47.025) (width 0.8) (layer "F.Cu") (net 9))
 (segment (start 213.895 47.165) (end 213.755 47.025) (width 0.8) (layer "F.Cu") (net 9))
 (segment (start 164.395 51.835) (end 164.395 47.165) (width 0.8) (layer "F.Cu") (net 9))
 (segment (start 213.895 51.835) (end 213.895 47.165) (width 0.8) (layer "F.Cu") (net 9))
 (segment (start 166.795 47.025) (end 166.795 51.695) (width 0.8) (layer "F.Cu") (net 8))
 (segment (start 166.795 51.695) (end 166.935 51.835) (width 0.8) (layer "F.Cu") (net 8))
 (segment (start 216.295 51.695) (end 216.435 51.835) (width 0.8) (layer "F.Cu") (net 8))
 (segment (start 216.295 47.025) (end 216.295 51.695) (width 0.8) (layer "F.Cu") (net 8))
 (segment (start 169.335 59.915) (end 169.475 59.775) (width 0.8) (layer "F.Cu") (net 18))
 (segment (start 218.835 59.915) (end 218.975 59.775) (width 0.8) (layer "F.Cu") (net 18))
 (segment (start 218.835 64.275) (end 218.835 59.915) (width 0.8) (layer "F.Cu") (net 18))
 (segment (start 169.335 64.275) (end 169.335 59.915) (width 0.8) (layer "F.Cu") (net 18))
 (segment (start 211.12 57) (end 213.895 59.775) (width 0.8) (layer "F.Cu") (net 16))
 (segment (start 164.255 59.915) (end 164.395 59.775) (width 0.8) (layer "F.Cu") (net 16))
 (segment (start 213.755 64.275) (end 213.755 59.915) (width 0.8) (layer "F.Cu") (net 16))
 (segment (start 197.75 57) (end 211.12 57) (width 0.8) (layer "F.Cu") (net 16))
 (segment (start 161.62 57) (end 164.395 59.775) (width 0.8) (layer "F.Cu") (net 16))
 (segment (start 197 60.46) (end 197 57.75) (width 0.8) (layer "F.Cu") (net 16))
 (segment (start 197 57.75) (end 197.75 57) (width 0.8) (layer "F.Cu") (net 16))
 (segment (start 148.25 57) (end 161.62 57) (width 0.8) (layer "F.Cu") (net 16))
 (segment (start 147.5 60.46) (end 147.5 57.75) (width 0.8) (layer "F.Cu") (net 16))
 (segment (start 213.755 59.915) (end 213.895 59.775) (width 0.8) (layer "F.Cu") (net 16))
 (segment (start 164.255 64.275) (end 164.255 59.915) (width 0.8) (layer "F.Cu") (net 16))
 (segment (start 147.5 57.75) (end 148.25 57) (width 0.8) (layer "F.Cu") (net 16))
 (segment (start 171.875 59.915) (end 172.015 59.775) (width 0.8) (layer "F.Cu") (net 19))
 (segment (start 171.875 64.275) (end 171.875 59.915) (width 0.8) (layer "F.Cu") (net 19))
 (segment (start 221.375 59.915) (end 221.515 59.775) (width 0.8) (layer "F.Cu") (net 19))
 (segment (start 221.375 64.275) (end 221.375 59.915) (width 0.8) (layer "F.Cu") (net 19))
 (segment (start 196.5 52.75) (end 196.5 55.25) (width 0.8) (layer "F.Cu") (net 3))
 (segment (start 146.25 63) (end 147.5 63) (width 0.8) (layer "F.Cu") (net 3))
 (segment (start 147.5 63) (end 147.5 66.25) (width 0.8) (layer "F.Cu") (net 3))
 (segment (start 150.975 64.275) (end 148.25 67) (width 0.8) (layer "F.Cu") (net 3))
 (segment (start 203.595 64.275) (end 200.475 64.275) (width 0.8) (layer "F.Cu") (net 3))
 (segment (start 196.25 53.0759) (end 196.25 47) (width 0.8) (layer "F.Cu") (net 3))
 (segment (start 147 52.75) (end 147 55.25) (width 0.8) (layer "F.Cu") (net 3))
 (segment (start 154.235 59.775) (end 154.095 59.915) (width 0.8) (layer "F.Cu") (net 3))
 (segment (start 147 55.25) (end 143.5 58.75) (width 0.8) (layer "F.Cu") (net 3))
 (segment (start 196.5 53.3259) (end 196.25 53.0759) (width 0.8) (layer "F.Cu") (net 3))
 (segment (start 203.595 59.915) (end 203.595 64.275) (width 0.8) (layer "F.Cu") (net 3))
 (segment (start 193 60.25) (end 195.75 63) (width 0.8) (layer "F.Cu") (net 3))
 (segment (start 143.5 58.75) (end 143.5 60.25) (width 0.8) (layer "F.Cu") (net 3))
 (segment (start 146.75 53.0759) (end 146.75 47) (width 0.8) (layer "F.Cu") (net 3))
 (segment (start 196.5 52.75) (end 196.5 53.3259) (width 0.8) (layer "F.Cu") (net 3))
 (segment (start 154.095 59.915) (end 154.095 64.275) (width 0.8) (layer "F.Cu") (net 3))
 (segment (start 147.5 66.25) (end 148.25 67) (width 0.8) (layer "F.Cu") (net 3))
 (segment (start 197 66.25) (end 197.75 67) (width 0.8) (layer "F.Cu") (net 3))
 (segment (start 203.735 59.775) (end 203.595 59.915) (width 0.8) (layer "F.Cu") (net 3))
 (segment (start 193 58.75) (end 193 60.25) (width 0.8) (layer "F.Cu") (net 3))
 (segment (start 195.75 63) (end 197 63) (width 0.8) (layer "F.Cu") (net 3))
 (segment (start 154.095 64.275) (end 150.975 64.275) (width 0.8) (layer "F.Cu") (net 3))
 (segment (start 197 63) (end 197 66.25) (width 0.8) (layer "F.Cu") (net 3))
 (segment (start 143.5 60.25) (end 146.25 63) (width 0.8) (layer "F.Cu") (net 3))
 (segment (start 147 53.3259) (end 146.75 53.0759) (width 0.8) (layer "F.Cu") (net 3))
 (segment (start 147 52.75) (end 147 53.3259) (width 0.8) (layer "F.Cu") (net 3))
 (segment (start 196.5 55.25) (end 193 58.75) (width 0.8) (layer "F.Cu") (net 3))
 (segment (start 200.475 64.275) (end 197.75 67) (width 0.8) (layer "F.Cu") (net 3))
 (segment (start 188.75 52.75) (end 193.96 52.75) (width 0.8) (layer "F.Cu") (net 6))
 (segment (start 139.25 52.75) (end 144.46 52.75) (width 0.8) (layer "F.Cu") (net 6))
 (segment (start 140 66.275) (end 144.985 66.275) (width 0.8) (layer "F.Cu") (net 5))
 (segment (start 189.5 66.275) (end 194.485 66.275) (width 0.8) (layer "F.Cu") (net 5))
 (segment (start 194.485 66.275) (end 195.21 67) (width 0.8) (layer "F.Cu") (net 5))
 (segment (start 144.985 66.275) (end 145.71 67) (width 0.8) (layer "F.Cu") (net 5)))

